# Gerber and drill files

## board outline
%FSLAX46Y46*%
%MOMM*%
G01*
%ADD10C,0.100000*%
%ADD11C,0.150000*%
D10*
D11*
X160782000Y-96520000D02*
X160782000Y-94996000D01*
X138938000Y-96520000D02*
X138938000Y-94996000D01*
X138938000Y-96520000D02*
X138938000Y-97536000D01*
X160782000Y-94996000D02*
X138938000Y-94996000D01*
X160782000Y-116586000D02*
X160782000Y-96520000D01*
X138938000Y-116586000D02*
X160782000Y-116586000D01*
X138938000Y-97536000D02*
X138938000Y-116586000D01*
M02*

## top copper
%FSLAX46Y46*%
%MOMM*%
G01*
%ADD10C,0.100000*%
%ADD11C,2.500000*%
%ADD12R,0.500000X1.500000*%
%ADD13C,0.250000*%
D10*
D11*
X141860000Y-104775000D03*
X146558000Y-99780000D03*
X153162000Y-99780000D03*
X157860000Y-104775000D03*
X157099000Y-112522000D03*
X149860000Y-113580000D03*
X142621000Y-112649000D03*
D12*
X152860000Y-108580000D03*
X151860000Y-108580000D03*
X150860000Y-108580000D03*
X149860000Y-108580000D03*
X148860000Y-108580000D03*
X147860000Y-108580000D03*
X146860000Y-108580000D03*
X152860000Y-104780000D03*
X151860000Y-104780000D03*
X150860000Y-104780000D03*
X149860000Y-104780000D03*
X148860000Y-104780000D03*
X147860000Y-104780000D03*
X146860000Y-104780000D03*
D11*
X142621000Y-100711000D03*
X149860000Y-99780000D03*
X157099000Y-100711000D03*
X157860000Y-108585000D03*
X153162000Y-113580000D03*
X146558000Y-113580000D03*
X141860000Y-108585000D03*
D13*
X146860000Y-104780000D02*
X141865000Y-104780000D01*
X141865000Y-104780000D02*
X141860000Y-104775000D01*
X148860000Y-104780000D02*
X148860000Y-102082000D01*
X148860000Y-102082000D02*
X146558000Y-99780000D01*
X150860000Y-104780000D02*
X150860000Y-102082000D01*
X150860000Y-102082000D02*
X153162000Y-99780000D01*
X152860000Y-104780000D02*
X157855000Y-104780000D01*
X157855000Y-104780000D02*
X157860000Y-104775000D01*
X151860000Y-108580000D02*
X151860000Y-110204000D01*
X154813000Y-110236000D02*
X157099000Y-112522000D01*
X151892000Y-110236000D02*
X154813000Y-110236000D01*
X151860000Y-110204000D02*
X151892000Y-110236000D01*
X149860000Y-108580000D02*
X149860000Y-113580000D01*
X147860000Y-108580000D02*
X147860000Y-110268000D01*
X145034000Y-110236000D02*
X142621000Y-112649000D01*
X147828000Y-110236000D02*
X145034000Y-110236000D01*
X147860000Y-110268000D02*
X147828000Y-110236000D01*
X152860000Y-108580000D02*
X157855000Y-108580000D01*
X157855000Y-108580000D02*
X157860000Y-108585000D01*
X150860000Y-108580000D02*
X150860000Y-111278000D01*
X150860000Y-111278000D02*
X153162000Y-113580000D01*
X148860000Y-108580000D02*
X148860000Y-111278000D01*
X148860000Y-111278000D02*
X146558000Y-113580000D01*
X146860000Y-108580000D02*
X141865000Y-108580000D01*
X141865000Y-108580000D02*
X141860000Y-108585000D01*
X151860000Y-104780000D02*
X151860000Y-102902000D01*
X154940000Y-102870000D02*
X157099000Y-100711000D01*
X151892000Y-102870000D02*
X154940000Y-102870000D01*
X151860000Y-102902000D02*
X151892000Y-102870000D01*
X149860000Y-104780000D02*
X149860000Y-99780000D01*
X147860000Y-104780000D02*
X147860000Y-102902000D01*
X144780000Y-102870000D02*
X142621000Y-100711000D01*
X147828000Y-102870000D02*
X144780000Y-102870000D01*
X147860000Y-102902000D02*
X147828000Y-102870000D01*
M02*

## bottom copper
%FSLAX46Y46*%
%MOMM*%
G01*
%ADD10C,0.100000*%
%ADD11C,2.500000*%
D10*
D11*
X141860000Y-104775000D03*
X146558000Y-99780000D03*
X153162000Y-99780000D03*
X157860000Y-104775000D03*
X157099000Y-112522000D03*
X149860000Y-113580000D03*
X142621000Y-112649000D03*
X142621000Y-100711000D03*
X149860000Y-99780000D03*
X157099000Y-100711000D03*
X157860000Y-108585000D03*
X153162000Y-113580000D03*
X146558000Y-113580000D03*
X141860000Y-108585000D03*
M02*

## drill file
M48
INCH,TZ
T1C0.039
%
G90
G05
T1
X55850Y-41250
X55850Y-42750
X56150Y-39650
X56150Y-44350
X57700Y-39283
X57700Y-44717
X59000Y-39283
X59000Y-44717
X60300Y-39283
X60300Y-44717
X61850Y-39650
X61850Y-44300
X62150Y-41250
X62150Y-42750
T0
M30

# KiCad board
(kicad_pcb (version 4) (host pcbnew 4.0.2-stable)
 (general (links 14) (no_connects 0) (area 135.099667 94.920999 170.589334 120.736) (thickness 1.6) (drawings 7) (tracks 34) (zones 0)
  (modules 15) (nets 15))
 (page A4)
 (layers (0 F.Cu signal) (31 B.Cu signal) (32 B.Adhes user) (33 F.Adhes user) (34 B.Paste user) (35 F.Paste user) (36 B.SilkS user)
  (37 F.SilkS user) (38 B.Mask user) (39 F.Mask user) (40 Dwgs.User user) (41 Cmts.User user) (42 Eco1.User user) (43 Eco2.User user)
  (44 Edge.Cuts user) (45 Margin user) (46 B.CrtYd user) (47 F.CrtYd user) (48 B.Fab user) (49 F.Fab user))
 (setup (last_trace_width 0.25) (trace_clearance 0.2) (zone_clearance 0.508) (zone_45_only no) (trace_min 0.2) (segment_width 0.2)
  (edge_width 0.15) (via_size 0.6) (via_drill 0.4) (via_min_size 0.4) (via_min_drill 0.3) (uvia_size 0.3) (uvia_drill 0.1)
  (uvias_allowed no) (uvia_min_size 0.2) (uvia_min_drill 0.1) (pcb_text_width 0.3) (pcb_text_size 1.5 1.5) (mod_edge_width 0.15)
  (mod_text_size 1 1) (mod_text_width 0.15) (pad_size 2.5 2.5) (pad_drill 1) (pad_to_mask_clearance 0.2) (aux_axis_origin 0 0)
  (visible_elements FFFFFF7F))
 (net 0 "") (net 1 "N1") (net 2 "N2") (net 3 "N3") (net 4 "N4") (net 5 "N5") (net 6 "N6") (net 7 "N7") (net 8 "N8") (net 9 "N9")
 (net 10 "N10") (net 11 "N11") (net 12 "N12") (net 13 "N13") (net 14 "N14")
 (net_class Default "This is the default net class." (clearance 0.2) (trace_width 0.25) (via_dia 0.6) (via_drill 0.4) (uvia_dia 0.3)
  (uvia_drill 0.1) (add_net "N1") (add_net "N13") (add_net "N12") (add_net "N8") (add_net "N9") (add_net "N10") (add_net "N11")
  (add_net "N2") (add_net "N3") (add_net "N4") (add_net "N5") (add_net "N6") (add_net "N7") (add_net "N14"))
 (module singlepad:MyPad (layer F.Cu) (at 140.208 108.585)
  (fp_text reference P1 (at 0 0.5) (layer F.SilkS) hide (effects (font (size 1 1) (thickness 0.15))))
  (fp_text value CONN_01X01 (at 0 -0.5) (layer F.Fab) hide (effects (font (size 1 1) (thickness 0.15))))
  (pad 1 thru_hole circle (at 1.652 -3.81) (size 2.5 2.5) (drill 1) (layers *.Cu *.Mask F.SilkS) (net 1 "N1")))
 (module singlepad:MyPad (layer F.Cu) (at 145.288 104.14)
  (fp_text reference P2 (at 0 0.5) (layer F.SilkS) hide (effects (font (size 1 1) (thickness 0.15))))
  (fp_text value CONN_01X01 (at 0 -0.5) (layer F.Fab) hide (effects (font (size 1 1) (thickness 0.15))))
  (pad 1 thru_hole circle (at 1.27 -4.36) (size 2.5 2.5) (drill 1) (layers *.Cu *.Mask F.SilkS) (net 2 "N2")))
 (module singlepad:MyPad (layer F.Cu) (at 151.892 104.14)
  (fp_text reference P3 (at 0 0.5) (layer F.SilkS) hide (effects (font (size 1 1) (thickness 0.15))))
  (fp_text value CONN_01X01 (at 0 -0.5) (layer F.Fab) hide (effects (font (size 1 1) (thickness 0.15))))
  (pad 1 thru_hole circle (at 1.27 -4.36) (size 2.5 2.5) (drill 1) (layers *.Cu *.Mask F.SilkS) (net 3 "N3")))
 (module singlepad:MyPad (layer F.Cu) (at 157.861 108.585)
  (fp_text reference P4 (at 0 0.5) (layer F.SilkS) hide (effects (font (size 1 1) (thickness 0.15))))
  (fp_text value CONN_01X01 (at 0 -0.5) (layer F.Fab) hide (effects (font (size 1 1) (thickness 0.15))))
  (pad 1 thru_hole circle (at -0.001 -3.81) (size 2.5 2.5) (drill 1) (layers *.Cu *.Mask F.SilkS) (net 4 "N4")))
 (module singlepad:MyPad (layer F.Cu) (at 156.337 116.332)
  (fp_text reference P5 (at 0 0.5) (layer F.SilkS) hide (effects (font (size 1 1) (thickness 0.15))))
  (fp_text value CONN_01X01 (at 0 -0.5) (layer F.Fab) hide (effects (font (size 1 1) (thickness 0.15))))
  (pad 1 thru_hole circle (at 0.762 -3.81) (size 2.5 2.5) (drill 1) (layers *.Cu *.Mask F.SilkS) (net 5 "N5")))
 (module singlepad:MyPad (layer F.Cu) (at 148.59 117.221)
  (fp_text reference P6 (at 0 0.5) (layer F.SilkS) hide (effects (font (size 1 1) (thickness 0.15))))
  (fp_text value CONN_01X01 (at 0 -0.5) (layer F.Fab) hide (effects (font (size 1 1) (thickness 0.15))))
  (pad 1 thru_hole circle (at 1.27 -3.641) (size 2.5 2.5) (drill 1) (layers *.Cu *.Mask F.SilkS) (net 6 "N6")))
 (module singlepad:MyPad (layer F.Cu) (at 140.589 116.459)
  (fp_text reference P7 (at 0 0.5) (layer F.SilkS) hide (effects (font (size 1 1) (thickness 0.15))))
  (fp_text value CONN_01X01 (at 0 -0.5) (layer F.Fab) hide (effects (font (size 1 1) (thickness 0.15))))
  (pad 1 thru_hole circle (at 2.032 -3.81) (size 2.5 2.5) (drill 1) (layers *.Cu *.Mask F.SilkS) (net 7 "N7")))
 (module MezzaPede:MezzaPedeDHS (layer F.Cu) (at 149.86 106.68)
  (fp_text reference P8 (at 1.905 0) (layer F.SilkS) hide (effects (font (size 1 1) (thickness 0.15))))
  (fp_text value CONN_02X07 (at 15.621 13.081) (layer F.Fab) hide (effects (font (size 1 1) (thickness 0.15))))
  (pad 8 smd rect (at 3 1.9) (size 0.5 1.5) (layers F.Cu F.Paste F.Mask) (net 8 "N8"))
  (pad 9 smd rect (at 2 1.9) (size 0.5 1.5) (layers F.Cu F.Paste F.Mask) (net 5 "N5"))
  (pad 10 smd rect (at 1 1.9) (size 0.5 1.5) (layers F.Cu F.Paste F.Mask) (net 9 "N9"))
  (pad 11 smd rect (at 0 1.9) (size 0.5 1.5) (layers F.Cu F.Paste F.Mask) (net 6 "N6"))
  (pad 12 smd rect (at -1 1.9) (size 0.5 1.5) (layers F.Cu F.Paste F.Mask) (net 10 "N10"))
  (pad 13 smd rect (at -2 1.9) (size 0.5 1.5) (layers F.Cu F.Paste F.Mask) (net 7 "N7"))
  (pad 14 smd rect (at -3 1.9) (size 0.5 1.5) (layers F.Cu F.Paste F.Mask) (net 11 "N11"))
  (pad 7 smd rect (at 3 -1.9) (size 0.5 1.5) (layers F.Cu F.Paste F.Mask) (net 4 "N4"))
  (pad 6 smd rect (at 2 -1.9) (size 0.5 1.5) (layers F.Cu F.Paste F.Mask) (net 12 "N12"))
  (pad 5 smd rect (at 1 -1.9) (size 0.5 1.5) (layers F.Cu F.Paste F.Mask) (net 3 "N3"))
  (pad 4 smd rect (at 0 -1.9) (size 0.5 1.5) (layers F.Cu F.Paste F.Mask) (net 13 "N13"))
  (pad 3 smd rect (at -1 -1.9) (size 0.5 1.5) (layers F.Cu F.Paste F.Mask) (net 2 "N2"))
  (pad 2 smd rect (at -2 -1.9) (size 0.5 1.5) (layers F.Cu F.Paste F.Mask) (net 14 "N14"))
  (pad 1 smd rect (at -3 -1.9) (size 0.5 1.5) (layers F.Cu F.Paste F.Mask) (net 1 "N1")))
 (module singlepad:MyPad (layer F.Cu) (at 141.351 104.521)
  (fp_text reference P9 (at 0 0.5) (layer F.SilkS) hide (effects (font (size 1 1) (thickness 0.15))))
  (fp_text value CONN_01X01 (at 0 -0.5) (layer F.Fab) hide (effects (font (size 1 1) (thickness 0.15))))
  (pad 1 thru_hole circle (at 1.27 -3.81) (size 2.5 2.5) (drill 1) (layers *.Cu *.Mask F.SilkS) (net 14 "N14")))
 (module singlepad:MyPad (layer F.Cu) (at 148.59 104.013)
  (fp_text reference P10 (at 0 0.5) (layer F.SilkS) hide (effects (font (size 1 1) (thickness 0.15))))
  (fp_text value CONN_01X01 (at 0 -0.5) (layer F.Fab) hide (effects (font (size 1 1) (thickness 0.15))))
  (pad 1 thru_hole circle (at 1.27 -4.233) (size 2.5 2.5) (drill 1) (layers *.Cu *.Mask F.SilkS) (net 13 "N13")))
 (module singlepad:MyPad (layer F.Cu) (at 155.829 104.14)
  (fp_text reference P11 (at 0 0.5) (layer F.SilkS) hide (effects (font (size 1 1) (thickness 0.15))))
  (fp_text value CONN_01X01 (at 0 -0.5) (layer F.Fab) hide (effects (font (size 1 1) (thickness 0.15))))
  (pad 1 thru_hole circle (at 1.27 -3.429) (size 2.5 2.5) (drill 1) (layers *.Cu *.Mask F.SilkS) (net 12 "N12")))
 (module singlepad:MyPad (layer F.Cu) (at 157.861 112.395)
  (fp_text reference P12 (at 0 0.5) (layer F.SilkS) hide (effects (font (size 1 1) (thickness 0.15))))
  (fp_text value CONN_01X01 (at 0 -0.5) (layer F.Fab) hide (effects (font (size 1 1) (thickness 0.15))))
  (pad 1 thru_hole circle (at -0.001 -3.81) (size 2.5 2.5) (drill 1) (layers *.Cu *.Mask F.SilkS) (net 8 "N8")))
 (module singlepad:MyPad (layer F.Cu) (at 151.892 117.475)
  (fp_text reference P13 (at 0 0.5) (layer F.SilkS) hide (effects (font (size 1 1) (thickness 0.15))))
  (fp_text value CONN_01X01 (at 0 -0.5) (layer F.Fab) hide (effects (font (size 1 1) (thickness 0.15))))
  (pad 1 thru_hole circle (at 1.27 -3.895) (size 2.5 2.5) (drill 1) (layers *.Cu *.Mask F.SilkS) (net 9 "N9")))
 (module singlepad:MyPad (layer F.Cu) (at 145.288 117.094)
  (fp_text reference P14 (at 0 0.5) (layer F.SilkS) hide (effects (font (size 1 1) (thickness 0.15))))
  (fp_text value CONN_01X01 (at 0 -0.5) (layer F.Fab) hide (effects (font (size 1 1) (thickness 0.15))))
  (pad 1 thru_hole circle (at 1.27 -3.514) (size 2.5 2.5) (drill 1) (layers *.Cu *.Mask F.SilkS) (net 10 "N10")))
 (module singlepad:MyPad (layer F.Cu) (at 140.208 112.395)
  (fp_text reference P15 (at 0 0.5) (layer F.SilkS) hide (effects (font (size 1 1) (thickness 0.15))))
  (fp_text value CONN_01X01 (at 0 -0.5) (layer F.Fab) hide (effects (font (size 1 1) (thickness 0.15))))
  (pad 1 thru_hole circle (at 1.652 -3.81) (size 2.5 2.5) (drill 1) (layers *.Cu *.Mask F.SilkS) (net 11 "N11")))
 (gr_line (start 160.782 96.52) (end 160.782 94.996) (angle 90) (layer Edge.Cuts) (width 0.15))
 (gr_line (start 138.938 96.52) (end 138.938 94.996) (angle 90) (layer Edge.Cuts) (width 0.15))
 (gr_line (start 138.938 96.52) (end 138.938 97.536) (angle 90) (layer Edge.Cuts) (width 0.15))
 (gr_line (start 160.782 94.996) (end 138.938 94.996) (angle 90) (layer Edge.Cuts) (width 0.15))
 (gr_line (start 160.782 116.586) (end 160.782 96.52) (angle 90) (layer Edge.Cuts) (width 0.15))
 (gr_line (start 138.938 116.586) (end 160.782 116.586) (angle 90) (layer Edge.Cuts) (width 0.15))
 (gr_line (start 138.938 97.536) (end 138.938 116.586) (angle 90) (layer Edge.Cuts) (width 0.15))
 (segment (start 146.86 104.78) (end 141.865 104.78) (width 0.25) (layer F.Cu) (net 1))
 (segment (start 141.865 104.78) (end 141.86 104.775) (width 0.25) (layer F.Cu) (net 1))
 (segment (start 148.86 104.78) (end 148.86 102.082) (width 0.25) (layer F.Cu) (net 2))
 (segment (start 148.86 102.082) (end 146.558 99.78) (width 0.25) (layer F.Cu) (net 2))
 (segment (start 150.86 104.78) (end 150.86 102.082) (width 0.25) (layer F.Cu) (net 3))
 (segment (start 150.86 102.082) (end 153.162 99.78) (width 0.25) (layer F.Cu) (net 3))
 (segment (start 152.86 104.78) (end 157.855 104.78) (width 0.25) (layer F.Cu) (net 4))
 (segment (start 157.855 104.78) (end 157.86 104.775) (width 0.25) (layer F.Cu) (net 4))
 (segment (start 151.86 108.58) (end 151.86 110.204) (width 0.25) (layer F.Cu) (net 5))
 (segment (start 154.813 110.236) (end 157.099 112.522) (width 0.25) (layer F.Cu) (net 5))
 (segment (start 151.892 110.236) (end 154.813 110.236) (width 0.25) (layer F.Cu) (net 5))
 (segment (start 151.86 110.204) (end 151.892 110.236) (width 0.25) (layer F.Cu) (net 5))
 (segment (start 149.86 108.58) (end 149.86 113.58) (width 0.25) (layer F.Cu) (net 6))
 (segment (start 147.86 108.58) (end 147.86 110.268) (width 0.25) (layer F.Cu) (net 7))
 (segment (start 145.034 110.236) (end 142.621 112.649) (width 0.25) (layer F.Cu) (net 7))
 (segment (start 147.828 110.236) (end 145.034 110.236) (width 0.25) (layer F.Cu) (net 7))
 (segment (start 147.86 110.268) (end 147.828 110.236) (width 0.25) (layer F.Cu) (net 7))
 (segment (start 152.86 108.58) (end 157.855 108.58) (width 0.25) (layer F.Cu) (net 8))
 (segment (start 157.855 108.58) (end 157.86 108.585) (width 0.25) (layer F.Cu) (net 8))
 (segment (start 150.86 108.58) (end 150.86 111.278) (width 0.25) (layer F.Cu) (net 9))
 (segment (start 150.86 111.278) (end 153.162 113.58) (width 0.25) (layer F.Cu) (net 9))
 (segment (start 148.86 108.58) (end 148.86 111.278) (width 0.25) (layer F.Cu) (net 10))
 (segment (start 148.86 111.278) (end 146.558 113.58) (width 0.25) (layer F.Cu) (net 10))
 (segment (start 146.86 108.58) (end 141.865 108.58) (width 0.25) (layer F.Cu) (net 11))
 (segment (start 141.865 108.58) (end 141.86 108.585) (width 0.25) (layer F.Cu) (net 11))
 (segment (start 151.86 104.78) (end 151.86 102.902) (width 0.25) (layer F.Cu) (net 12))
 (segment (start 154.94 102.87) (end 157.099 100.711) (width 0.25) (layer F.Cu) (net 12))
 (segment (start 151.892 102.87) (end 154.94 102.87) (width 0.25) (layer F.Cu) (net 12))
 (segment (start 151.86 102.902) (end 151.892 102.87) (width 0.25) (layer F.Cu) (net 12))
 (segment (start 149.86 104.78) (end 149.86 99.78) (width 0.25) (layer F.Cu) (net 13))
 (segment (start 147.86 104.78) (end 147.86 102.902) (width 0.25) (layer F.Cu) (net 14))
 (segment (start 144.78 102.87) (end 142.621 100.711) (width 0.25) (layer F.Cu) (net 14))
 (segment (start 147.828 102.87) (end 144.78 102.87) (width 0.25) (layer F.Cu) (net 14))
 (segment (start 147.86 102.902) (end 147.828 102.87) (width 0.25) (layer F.Cu) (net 14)))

